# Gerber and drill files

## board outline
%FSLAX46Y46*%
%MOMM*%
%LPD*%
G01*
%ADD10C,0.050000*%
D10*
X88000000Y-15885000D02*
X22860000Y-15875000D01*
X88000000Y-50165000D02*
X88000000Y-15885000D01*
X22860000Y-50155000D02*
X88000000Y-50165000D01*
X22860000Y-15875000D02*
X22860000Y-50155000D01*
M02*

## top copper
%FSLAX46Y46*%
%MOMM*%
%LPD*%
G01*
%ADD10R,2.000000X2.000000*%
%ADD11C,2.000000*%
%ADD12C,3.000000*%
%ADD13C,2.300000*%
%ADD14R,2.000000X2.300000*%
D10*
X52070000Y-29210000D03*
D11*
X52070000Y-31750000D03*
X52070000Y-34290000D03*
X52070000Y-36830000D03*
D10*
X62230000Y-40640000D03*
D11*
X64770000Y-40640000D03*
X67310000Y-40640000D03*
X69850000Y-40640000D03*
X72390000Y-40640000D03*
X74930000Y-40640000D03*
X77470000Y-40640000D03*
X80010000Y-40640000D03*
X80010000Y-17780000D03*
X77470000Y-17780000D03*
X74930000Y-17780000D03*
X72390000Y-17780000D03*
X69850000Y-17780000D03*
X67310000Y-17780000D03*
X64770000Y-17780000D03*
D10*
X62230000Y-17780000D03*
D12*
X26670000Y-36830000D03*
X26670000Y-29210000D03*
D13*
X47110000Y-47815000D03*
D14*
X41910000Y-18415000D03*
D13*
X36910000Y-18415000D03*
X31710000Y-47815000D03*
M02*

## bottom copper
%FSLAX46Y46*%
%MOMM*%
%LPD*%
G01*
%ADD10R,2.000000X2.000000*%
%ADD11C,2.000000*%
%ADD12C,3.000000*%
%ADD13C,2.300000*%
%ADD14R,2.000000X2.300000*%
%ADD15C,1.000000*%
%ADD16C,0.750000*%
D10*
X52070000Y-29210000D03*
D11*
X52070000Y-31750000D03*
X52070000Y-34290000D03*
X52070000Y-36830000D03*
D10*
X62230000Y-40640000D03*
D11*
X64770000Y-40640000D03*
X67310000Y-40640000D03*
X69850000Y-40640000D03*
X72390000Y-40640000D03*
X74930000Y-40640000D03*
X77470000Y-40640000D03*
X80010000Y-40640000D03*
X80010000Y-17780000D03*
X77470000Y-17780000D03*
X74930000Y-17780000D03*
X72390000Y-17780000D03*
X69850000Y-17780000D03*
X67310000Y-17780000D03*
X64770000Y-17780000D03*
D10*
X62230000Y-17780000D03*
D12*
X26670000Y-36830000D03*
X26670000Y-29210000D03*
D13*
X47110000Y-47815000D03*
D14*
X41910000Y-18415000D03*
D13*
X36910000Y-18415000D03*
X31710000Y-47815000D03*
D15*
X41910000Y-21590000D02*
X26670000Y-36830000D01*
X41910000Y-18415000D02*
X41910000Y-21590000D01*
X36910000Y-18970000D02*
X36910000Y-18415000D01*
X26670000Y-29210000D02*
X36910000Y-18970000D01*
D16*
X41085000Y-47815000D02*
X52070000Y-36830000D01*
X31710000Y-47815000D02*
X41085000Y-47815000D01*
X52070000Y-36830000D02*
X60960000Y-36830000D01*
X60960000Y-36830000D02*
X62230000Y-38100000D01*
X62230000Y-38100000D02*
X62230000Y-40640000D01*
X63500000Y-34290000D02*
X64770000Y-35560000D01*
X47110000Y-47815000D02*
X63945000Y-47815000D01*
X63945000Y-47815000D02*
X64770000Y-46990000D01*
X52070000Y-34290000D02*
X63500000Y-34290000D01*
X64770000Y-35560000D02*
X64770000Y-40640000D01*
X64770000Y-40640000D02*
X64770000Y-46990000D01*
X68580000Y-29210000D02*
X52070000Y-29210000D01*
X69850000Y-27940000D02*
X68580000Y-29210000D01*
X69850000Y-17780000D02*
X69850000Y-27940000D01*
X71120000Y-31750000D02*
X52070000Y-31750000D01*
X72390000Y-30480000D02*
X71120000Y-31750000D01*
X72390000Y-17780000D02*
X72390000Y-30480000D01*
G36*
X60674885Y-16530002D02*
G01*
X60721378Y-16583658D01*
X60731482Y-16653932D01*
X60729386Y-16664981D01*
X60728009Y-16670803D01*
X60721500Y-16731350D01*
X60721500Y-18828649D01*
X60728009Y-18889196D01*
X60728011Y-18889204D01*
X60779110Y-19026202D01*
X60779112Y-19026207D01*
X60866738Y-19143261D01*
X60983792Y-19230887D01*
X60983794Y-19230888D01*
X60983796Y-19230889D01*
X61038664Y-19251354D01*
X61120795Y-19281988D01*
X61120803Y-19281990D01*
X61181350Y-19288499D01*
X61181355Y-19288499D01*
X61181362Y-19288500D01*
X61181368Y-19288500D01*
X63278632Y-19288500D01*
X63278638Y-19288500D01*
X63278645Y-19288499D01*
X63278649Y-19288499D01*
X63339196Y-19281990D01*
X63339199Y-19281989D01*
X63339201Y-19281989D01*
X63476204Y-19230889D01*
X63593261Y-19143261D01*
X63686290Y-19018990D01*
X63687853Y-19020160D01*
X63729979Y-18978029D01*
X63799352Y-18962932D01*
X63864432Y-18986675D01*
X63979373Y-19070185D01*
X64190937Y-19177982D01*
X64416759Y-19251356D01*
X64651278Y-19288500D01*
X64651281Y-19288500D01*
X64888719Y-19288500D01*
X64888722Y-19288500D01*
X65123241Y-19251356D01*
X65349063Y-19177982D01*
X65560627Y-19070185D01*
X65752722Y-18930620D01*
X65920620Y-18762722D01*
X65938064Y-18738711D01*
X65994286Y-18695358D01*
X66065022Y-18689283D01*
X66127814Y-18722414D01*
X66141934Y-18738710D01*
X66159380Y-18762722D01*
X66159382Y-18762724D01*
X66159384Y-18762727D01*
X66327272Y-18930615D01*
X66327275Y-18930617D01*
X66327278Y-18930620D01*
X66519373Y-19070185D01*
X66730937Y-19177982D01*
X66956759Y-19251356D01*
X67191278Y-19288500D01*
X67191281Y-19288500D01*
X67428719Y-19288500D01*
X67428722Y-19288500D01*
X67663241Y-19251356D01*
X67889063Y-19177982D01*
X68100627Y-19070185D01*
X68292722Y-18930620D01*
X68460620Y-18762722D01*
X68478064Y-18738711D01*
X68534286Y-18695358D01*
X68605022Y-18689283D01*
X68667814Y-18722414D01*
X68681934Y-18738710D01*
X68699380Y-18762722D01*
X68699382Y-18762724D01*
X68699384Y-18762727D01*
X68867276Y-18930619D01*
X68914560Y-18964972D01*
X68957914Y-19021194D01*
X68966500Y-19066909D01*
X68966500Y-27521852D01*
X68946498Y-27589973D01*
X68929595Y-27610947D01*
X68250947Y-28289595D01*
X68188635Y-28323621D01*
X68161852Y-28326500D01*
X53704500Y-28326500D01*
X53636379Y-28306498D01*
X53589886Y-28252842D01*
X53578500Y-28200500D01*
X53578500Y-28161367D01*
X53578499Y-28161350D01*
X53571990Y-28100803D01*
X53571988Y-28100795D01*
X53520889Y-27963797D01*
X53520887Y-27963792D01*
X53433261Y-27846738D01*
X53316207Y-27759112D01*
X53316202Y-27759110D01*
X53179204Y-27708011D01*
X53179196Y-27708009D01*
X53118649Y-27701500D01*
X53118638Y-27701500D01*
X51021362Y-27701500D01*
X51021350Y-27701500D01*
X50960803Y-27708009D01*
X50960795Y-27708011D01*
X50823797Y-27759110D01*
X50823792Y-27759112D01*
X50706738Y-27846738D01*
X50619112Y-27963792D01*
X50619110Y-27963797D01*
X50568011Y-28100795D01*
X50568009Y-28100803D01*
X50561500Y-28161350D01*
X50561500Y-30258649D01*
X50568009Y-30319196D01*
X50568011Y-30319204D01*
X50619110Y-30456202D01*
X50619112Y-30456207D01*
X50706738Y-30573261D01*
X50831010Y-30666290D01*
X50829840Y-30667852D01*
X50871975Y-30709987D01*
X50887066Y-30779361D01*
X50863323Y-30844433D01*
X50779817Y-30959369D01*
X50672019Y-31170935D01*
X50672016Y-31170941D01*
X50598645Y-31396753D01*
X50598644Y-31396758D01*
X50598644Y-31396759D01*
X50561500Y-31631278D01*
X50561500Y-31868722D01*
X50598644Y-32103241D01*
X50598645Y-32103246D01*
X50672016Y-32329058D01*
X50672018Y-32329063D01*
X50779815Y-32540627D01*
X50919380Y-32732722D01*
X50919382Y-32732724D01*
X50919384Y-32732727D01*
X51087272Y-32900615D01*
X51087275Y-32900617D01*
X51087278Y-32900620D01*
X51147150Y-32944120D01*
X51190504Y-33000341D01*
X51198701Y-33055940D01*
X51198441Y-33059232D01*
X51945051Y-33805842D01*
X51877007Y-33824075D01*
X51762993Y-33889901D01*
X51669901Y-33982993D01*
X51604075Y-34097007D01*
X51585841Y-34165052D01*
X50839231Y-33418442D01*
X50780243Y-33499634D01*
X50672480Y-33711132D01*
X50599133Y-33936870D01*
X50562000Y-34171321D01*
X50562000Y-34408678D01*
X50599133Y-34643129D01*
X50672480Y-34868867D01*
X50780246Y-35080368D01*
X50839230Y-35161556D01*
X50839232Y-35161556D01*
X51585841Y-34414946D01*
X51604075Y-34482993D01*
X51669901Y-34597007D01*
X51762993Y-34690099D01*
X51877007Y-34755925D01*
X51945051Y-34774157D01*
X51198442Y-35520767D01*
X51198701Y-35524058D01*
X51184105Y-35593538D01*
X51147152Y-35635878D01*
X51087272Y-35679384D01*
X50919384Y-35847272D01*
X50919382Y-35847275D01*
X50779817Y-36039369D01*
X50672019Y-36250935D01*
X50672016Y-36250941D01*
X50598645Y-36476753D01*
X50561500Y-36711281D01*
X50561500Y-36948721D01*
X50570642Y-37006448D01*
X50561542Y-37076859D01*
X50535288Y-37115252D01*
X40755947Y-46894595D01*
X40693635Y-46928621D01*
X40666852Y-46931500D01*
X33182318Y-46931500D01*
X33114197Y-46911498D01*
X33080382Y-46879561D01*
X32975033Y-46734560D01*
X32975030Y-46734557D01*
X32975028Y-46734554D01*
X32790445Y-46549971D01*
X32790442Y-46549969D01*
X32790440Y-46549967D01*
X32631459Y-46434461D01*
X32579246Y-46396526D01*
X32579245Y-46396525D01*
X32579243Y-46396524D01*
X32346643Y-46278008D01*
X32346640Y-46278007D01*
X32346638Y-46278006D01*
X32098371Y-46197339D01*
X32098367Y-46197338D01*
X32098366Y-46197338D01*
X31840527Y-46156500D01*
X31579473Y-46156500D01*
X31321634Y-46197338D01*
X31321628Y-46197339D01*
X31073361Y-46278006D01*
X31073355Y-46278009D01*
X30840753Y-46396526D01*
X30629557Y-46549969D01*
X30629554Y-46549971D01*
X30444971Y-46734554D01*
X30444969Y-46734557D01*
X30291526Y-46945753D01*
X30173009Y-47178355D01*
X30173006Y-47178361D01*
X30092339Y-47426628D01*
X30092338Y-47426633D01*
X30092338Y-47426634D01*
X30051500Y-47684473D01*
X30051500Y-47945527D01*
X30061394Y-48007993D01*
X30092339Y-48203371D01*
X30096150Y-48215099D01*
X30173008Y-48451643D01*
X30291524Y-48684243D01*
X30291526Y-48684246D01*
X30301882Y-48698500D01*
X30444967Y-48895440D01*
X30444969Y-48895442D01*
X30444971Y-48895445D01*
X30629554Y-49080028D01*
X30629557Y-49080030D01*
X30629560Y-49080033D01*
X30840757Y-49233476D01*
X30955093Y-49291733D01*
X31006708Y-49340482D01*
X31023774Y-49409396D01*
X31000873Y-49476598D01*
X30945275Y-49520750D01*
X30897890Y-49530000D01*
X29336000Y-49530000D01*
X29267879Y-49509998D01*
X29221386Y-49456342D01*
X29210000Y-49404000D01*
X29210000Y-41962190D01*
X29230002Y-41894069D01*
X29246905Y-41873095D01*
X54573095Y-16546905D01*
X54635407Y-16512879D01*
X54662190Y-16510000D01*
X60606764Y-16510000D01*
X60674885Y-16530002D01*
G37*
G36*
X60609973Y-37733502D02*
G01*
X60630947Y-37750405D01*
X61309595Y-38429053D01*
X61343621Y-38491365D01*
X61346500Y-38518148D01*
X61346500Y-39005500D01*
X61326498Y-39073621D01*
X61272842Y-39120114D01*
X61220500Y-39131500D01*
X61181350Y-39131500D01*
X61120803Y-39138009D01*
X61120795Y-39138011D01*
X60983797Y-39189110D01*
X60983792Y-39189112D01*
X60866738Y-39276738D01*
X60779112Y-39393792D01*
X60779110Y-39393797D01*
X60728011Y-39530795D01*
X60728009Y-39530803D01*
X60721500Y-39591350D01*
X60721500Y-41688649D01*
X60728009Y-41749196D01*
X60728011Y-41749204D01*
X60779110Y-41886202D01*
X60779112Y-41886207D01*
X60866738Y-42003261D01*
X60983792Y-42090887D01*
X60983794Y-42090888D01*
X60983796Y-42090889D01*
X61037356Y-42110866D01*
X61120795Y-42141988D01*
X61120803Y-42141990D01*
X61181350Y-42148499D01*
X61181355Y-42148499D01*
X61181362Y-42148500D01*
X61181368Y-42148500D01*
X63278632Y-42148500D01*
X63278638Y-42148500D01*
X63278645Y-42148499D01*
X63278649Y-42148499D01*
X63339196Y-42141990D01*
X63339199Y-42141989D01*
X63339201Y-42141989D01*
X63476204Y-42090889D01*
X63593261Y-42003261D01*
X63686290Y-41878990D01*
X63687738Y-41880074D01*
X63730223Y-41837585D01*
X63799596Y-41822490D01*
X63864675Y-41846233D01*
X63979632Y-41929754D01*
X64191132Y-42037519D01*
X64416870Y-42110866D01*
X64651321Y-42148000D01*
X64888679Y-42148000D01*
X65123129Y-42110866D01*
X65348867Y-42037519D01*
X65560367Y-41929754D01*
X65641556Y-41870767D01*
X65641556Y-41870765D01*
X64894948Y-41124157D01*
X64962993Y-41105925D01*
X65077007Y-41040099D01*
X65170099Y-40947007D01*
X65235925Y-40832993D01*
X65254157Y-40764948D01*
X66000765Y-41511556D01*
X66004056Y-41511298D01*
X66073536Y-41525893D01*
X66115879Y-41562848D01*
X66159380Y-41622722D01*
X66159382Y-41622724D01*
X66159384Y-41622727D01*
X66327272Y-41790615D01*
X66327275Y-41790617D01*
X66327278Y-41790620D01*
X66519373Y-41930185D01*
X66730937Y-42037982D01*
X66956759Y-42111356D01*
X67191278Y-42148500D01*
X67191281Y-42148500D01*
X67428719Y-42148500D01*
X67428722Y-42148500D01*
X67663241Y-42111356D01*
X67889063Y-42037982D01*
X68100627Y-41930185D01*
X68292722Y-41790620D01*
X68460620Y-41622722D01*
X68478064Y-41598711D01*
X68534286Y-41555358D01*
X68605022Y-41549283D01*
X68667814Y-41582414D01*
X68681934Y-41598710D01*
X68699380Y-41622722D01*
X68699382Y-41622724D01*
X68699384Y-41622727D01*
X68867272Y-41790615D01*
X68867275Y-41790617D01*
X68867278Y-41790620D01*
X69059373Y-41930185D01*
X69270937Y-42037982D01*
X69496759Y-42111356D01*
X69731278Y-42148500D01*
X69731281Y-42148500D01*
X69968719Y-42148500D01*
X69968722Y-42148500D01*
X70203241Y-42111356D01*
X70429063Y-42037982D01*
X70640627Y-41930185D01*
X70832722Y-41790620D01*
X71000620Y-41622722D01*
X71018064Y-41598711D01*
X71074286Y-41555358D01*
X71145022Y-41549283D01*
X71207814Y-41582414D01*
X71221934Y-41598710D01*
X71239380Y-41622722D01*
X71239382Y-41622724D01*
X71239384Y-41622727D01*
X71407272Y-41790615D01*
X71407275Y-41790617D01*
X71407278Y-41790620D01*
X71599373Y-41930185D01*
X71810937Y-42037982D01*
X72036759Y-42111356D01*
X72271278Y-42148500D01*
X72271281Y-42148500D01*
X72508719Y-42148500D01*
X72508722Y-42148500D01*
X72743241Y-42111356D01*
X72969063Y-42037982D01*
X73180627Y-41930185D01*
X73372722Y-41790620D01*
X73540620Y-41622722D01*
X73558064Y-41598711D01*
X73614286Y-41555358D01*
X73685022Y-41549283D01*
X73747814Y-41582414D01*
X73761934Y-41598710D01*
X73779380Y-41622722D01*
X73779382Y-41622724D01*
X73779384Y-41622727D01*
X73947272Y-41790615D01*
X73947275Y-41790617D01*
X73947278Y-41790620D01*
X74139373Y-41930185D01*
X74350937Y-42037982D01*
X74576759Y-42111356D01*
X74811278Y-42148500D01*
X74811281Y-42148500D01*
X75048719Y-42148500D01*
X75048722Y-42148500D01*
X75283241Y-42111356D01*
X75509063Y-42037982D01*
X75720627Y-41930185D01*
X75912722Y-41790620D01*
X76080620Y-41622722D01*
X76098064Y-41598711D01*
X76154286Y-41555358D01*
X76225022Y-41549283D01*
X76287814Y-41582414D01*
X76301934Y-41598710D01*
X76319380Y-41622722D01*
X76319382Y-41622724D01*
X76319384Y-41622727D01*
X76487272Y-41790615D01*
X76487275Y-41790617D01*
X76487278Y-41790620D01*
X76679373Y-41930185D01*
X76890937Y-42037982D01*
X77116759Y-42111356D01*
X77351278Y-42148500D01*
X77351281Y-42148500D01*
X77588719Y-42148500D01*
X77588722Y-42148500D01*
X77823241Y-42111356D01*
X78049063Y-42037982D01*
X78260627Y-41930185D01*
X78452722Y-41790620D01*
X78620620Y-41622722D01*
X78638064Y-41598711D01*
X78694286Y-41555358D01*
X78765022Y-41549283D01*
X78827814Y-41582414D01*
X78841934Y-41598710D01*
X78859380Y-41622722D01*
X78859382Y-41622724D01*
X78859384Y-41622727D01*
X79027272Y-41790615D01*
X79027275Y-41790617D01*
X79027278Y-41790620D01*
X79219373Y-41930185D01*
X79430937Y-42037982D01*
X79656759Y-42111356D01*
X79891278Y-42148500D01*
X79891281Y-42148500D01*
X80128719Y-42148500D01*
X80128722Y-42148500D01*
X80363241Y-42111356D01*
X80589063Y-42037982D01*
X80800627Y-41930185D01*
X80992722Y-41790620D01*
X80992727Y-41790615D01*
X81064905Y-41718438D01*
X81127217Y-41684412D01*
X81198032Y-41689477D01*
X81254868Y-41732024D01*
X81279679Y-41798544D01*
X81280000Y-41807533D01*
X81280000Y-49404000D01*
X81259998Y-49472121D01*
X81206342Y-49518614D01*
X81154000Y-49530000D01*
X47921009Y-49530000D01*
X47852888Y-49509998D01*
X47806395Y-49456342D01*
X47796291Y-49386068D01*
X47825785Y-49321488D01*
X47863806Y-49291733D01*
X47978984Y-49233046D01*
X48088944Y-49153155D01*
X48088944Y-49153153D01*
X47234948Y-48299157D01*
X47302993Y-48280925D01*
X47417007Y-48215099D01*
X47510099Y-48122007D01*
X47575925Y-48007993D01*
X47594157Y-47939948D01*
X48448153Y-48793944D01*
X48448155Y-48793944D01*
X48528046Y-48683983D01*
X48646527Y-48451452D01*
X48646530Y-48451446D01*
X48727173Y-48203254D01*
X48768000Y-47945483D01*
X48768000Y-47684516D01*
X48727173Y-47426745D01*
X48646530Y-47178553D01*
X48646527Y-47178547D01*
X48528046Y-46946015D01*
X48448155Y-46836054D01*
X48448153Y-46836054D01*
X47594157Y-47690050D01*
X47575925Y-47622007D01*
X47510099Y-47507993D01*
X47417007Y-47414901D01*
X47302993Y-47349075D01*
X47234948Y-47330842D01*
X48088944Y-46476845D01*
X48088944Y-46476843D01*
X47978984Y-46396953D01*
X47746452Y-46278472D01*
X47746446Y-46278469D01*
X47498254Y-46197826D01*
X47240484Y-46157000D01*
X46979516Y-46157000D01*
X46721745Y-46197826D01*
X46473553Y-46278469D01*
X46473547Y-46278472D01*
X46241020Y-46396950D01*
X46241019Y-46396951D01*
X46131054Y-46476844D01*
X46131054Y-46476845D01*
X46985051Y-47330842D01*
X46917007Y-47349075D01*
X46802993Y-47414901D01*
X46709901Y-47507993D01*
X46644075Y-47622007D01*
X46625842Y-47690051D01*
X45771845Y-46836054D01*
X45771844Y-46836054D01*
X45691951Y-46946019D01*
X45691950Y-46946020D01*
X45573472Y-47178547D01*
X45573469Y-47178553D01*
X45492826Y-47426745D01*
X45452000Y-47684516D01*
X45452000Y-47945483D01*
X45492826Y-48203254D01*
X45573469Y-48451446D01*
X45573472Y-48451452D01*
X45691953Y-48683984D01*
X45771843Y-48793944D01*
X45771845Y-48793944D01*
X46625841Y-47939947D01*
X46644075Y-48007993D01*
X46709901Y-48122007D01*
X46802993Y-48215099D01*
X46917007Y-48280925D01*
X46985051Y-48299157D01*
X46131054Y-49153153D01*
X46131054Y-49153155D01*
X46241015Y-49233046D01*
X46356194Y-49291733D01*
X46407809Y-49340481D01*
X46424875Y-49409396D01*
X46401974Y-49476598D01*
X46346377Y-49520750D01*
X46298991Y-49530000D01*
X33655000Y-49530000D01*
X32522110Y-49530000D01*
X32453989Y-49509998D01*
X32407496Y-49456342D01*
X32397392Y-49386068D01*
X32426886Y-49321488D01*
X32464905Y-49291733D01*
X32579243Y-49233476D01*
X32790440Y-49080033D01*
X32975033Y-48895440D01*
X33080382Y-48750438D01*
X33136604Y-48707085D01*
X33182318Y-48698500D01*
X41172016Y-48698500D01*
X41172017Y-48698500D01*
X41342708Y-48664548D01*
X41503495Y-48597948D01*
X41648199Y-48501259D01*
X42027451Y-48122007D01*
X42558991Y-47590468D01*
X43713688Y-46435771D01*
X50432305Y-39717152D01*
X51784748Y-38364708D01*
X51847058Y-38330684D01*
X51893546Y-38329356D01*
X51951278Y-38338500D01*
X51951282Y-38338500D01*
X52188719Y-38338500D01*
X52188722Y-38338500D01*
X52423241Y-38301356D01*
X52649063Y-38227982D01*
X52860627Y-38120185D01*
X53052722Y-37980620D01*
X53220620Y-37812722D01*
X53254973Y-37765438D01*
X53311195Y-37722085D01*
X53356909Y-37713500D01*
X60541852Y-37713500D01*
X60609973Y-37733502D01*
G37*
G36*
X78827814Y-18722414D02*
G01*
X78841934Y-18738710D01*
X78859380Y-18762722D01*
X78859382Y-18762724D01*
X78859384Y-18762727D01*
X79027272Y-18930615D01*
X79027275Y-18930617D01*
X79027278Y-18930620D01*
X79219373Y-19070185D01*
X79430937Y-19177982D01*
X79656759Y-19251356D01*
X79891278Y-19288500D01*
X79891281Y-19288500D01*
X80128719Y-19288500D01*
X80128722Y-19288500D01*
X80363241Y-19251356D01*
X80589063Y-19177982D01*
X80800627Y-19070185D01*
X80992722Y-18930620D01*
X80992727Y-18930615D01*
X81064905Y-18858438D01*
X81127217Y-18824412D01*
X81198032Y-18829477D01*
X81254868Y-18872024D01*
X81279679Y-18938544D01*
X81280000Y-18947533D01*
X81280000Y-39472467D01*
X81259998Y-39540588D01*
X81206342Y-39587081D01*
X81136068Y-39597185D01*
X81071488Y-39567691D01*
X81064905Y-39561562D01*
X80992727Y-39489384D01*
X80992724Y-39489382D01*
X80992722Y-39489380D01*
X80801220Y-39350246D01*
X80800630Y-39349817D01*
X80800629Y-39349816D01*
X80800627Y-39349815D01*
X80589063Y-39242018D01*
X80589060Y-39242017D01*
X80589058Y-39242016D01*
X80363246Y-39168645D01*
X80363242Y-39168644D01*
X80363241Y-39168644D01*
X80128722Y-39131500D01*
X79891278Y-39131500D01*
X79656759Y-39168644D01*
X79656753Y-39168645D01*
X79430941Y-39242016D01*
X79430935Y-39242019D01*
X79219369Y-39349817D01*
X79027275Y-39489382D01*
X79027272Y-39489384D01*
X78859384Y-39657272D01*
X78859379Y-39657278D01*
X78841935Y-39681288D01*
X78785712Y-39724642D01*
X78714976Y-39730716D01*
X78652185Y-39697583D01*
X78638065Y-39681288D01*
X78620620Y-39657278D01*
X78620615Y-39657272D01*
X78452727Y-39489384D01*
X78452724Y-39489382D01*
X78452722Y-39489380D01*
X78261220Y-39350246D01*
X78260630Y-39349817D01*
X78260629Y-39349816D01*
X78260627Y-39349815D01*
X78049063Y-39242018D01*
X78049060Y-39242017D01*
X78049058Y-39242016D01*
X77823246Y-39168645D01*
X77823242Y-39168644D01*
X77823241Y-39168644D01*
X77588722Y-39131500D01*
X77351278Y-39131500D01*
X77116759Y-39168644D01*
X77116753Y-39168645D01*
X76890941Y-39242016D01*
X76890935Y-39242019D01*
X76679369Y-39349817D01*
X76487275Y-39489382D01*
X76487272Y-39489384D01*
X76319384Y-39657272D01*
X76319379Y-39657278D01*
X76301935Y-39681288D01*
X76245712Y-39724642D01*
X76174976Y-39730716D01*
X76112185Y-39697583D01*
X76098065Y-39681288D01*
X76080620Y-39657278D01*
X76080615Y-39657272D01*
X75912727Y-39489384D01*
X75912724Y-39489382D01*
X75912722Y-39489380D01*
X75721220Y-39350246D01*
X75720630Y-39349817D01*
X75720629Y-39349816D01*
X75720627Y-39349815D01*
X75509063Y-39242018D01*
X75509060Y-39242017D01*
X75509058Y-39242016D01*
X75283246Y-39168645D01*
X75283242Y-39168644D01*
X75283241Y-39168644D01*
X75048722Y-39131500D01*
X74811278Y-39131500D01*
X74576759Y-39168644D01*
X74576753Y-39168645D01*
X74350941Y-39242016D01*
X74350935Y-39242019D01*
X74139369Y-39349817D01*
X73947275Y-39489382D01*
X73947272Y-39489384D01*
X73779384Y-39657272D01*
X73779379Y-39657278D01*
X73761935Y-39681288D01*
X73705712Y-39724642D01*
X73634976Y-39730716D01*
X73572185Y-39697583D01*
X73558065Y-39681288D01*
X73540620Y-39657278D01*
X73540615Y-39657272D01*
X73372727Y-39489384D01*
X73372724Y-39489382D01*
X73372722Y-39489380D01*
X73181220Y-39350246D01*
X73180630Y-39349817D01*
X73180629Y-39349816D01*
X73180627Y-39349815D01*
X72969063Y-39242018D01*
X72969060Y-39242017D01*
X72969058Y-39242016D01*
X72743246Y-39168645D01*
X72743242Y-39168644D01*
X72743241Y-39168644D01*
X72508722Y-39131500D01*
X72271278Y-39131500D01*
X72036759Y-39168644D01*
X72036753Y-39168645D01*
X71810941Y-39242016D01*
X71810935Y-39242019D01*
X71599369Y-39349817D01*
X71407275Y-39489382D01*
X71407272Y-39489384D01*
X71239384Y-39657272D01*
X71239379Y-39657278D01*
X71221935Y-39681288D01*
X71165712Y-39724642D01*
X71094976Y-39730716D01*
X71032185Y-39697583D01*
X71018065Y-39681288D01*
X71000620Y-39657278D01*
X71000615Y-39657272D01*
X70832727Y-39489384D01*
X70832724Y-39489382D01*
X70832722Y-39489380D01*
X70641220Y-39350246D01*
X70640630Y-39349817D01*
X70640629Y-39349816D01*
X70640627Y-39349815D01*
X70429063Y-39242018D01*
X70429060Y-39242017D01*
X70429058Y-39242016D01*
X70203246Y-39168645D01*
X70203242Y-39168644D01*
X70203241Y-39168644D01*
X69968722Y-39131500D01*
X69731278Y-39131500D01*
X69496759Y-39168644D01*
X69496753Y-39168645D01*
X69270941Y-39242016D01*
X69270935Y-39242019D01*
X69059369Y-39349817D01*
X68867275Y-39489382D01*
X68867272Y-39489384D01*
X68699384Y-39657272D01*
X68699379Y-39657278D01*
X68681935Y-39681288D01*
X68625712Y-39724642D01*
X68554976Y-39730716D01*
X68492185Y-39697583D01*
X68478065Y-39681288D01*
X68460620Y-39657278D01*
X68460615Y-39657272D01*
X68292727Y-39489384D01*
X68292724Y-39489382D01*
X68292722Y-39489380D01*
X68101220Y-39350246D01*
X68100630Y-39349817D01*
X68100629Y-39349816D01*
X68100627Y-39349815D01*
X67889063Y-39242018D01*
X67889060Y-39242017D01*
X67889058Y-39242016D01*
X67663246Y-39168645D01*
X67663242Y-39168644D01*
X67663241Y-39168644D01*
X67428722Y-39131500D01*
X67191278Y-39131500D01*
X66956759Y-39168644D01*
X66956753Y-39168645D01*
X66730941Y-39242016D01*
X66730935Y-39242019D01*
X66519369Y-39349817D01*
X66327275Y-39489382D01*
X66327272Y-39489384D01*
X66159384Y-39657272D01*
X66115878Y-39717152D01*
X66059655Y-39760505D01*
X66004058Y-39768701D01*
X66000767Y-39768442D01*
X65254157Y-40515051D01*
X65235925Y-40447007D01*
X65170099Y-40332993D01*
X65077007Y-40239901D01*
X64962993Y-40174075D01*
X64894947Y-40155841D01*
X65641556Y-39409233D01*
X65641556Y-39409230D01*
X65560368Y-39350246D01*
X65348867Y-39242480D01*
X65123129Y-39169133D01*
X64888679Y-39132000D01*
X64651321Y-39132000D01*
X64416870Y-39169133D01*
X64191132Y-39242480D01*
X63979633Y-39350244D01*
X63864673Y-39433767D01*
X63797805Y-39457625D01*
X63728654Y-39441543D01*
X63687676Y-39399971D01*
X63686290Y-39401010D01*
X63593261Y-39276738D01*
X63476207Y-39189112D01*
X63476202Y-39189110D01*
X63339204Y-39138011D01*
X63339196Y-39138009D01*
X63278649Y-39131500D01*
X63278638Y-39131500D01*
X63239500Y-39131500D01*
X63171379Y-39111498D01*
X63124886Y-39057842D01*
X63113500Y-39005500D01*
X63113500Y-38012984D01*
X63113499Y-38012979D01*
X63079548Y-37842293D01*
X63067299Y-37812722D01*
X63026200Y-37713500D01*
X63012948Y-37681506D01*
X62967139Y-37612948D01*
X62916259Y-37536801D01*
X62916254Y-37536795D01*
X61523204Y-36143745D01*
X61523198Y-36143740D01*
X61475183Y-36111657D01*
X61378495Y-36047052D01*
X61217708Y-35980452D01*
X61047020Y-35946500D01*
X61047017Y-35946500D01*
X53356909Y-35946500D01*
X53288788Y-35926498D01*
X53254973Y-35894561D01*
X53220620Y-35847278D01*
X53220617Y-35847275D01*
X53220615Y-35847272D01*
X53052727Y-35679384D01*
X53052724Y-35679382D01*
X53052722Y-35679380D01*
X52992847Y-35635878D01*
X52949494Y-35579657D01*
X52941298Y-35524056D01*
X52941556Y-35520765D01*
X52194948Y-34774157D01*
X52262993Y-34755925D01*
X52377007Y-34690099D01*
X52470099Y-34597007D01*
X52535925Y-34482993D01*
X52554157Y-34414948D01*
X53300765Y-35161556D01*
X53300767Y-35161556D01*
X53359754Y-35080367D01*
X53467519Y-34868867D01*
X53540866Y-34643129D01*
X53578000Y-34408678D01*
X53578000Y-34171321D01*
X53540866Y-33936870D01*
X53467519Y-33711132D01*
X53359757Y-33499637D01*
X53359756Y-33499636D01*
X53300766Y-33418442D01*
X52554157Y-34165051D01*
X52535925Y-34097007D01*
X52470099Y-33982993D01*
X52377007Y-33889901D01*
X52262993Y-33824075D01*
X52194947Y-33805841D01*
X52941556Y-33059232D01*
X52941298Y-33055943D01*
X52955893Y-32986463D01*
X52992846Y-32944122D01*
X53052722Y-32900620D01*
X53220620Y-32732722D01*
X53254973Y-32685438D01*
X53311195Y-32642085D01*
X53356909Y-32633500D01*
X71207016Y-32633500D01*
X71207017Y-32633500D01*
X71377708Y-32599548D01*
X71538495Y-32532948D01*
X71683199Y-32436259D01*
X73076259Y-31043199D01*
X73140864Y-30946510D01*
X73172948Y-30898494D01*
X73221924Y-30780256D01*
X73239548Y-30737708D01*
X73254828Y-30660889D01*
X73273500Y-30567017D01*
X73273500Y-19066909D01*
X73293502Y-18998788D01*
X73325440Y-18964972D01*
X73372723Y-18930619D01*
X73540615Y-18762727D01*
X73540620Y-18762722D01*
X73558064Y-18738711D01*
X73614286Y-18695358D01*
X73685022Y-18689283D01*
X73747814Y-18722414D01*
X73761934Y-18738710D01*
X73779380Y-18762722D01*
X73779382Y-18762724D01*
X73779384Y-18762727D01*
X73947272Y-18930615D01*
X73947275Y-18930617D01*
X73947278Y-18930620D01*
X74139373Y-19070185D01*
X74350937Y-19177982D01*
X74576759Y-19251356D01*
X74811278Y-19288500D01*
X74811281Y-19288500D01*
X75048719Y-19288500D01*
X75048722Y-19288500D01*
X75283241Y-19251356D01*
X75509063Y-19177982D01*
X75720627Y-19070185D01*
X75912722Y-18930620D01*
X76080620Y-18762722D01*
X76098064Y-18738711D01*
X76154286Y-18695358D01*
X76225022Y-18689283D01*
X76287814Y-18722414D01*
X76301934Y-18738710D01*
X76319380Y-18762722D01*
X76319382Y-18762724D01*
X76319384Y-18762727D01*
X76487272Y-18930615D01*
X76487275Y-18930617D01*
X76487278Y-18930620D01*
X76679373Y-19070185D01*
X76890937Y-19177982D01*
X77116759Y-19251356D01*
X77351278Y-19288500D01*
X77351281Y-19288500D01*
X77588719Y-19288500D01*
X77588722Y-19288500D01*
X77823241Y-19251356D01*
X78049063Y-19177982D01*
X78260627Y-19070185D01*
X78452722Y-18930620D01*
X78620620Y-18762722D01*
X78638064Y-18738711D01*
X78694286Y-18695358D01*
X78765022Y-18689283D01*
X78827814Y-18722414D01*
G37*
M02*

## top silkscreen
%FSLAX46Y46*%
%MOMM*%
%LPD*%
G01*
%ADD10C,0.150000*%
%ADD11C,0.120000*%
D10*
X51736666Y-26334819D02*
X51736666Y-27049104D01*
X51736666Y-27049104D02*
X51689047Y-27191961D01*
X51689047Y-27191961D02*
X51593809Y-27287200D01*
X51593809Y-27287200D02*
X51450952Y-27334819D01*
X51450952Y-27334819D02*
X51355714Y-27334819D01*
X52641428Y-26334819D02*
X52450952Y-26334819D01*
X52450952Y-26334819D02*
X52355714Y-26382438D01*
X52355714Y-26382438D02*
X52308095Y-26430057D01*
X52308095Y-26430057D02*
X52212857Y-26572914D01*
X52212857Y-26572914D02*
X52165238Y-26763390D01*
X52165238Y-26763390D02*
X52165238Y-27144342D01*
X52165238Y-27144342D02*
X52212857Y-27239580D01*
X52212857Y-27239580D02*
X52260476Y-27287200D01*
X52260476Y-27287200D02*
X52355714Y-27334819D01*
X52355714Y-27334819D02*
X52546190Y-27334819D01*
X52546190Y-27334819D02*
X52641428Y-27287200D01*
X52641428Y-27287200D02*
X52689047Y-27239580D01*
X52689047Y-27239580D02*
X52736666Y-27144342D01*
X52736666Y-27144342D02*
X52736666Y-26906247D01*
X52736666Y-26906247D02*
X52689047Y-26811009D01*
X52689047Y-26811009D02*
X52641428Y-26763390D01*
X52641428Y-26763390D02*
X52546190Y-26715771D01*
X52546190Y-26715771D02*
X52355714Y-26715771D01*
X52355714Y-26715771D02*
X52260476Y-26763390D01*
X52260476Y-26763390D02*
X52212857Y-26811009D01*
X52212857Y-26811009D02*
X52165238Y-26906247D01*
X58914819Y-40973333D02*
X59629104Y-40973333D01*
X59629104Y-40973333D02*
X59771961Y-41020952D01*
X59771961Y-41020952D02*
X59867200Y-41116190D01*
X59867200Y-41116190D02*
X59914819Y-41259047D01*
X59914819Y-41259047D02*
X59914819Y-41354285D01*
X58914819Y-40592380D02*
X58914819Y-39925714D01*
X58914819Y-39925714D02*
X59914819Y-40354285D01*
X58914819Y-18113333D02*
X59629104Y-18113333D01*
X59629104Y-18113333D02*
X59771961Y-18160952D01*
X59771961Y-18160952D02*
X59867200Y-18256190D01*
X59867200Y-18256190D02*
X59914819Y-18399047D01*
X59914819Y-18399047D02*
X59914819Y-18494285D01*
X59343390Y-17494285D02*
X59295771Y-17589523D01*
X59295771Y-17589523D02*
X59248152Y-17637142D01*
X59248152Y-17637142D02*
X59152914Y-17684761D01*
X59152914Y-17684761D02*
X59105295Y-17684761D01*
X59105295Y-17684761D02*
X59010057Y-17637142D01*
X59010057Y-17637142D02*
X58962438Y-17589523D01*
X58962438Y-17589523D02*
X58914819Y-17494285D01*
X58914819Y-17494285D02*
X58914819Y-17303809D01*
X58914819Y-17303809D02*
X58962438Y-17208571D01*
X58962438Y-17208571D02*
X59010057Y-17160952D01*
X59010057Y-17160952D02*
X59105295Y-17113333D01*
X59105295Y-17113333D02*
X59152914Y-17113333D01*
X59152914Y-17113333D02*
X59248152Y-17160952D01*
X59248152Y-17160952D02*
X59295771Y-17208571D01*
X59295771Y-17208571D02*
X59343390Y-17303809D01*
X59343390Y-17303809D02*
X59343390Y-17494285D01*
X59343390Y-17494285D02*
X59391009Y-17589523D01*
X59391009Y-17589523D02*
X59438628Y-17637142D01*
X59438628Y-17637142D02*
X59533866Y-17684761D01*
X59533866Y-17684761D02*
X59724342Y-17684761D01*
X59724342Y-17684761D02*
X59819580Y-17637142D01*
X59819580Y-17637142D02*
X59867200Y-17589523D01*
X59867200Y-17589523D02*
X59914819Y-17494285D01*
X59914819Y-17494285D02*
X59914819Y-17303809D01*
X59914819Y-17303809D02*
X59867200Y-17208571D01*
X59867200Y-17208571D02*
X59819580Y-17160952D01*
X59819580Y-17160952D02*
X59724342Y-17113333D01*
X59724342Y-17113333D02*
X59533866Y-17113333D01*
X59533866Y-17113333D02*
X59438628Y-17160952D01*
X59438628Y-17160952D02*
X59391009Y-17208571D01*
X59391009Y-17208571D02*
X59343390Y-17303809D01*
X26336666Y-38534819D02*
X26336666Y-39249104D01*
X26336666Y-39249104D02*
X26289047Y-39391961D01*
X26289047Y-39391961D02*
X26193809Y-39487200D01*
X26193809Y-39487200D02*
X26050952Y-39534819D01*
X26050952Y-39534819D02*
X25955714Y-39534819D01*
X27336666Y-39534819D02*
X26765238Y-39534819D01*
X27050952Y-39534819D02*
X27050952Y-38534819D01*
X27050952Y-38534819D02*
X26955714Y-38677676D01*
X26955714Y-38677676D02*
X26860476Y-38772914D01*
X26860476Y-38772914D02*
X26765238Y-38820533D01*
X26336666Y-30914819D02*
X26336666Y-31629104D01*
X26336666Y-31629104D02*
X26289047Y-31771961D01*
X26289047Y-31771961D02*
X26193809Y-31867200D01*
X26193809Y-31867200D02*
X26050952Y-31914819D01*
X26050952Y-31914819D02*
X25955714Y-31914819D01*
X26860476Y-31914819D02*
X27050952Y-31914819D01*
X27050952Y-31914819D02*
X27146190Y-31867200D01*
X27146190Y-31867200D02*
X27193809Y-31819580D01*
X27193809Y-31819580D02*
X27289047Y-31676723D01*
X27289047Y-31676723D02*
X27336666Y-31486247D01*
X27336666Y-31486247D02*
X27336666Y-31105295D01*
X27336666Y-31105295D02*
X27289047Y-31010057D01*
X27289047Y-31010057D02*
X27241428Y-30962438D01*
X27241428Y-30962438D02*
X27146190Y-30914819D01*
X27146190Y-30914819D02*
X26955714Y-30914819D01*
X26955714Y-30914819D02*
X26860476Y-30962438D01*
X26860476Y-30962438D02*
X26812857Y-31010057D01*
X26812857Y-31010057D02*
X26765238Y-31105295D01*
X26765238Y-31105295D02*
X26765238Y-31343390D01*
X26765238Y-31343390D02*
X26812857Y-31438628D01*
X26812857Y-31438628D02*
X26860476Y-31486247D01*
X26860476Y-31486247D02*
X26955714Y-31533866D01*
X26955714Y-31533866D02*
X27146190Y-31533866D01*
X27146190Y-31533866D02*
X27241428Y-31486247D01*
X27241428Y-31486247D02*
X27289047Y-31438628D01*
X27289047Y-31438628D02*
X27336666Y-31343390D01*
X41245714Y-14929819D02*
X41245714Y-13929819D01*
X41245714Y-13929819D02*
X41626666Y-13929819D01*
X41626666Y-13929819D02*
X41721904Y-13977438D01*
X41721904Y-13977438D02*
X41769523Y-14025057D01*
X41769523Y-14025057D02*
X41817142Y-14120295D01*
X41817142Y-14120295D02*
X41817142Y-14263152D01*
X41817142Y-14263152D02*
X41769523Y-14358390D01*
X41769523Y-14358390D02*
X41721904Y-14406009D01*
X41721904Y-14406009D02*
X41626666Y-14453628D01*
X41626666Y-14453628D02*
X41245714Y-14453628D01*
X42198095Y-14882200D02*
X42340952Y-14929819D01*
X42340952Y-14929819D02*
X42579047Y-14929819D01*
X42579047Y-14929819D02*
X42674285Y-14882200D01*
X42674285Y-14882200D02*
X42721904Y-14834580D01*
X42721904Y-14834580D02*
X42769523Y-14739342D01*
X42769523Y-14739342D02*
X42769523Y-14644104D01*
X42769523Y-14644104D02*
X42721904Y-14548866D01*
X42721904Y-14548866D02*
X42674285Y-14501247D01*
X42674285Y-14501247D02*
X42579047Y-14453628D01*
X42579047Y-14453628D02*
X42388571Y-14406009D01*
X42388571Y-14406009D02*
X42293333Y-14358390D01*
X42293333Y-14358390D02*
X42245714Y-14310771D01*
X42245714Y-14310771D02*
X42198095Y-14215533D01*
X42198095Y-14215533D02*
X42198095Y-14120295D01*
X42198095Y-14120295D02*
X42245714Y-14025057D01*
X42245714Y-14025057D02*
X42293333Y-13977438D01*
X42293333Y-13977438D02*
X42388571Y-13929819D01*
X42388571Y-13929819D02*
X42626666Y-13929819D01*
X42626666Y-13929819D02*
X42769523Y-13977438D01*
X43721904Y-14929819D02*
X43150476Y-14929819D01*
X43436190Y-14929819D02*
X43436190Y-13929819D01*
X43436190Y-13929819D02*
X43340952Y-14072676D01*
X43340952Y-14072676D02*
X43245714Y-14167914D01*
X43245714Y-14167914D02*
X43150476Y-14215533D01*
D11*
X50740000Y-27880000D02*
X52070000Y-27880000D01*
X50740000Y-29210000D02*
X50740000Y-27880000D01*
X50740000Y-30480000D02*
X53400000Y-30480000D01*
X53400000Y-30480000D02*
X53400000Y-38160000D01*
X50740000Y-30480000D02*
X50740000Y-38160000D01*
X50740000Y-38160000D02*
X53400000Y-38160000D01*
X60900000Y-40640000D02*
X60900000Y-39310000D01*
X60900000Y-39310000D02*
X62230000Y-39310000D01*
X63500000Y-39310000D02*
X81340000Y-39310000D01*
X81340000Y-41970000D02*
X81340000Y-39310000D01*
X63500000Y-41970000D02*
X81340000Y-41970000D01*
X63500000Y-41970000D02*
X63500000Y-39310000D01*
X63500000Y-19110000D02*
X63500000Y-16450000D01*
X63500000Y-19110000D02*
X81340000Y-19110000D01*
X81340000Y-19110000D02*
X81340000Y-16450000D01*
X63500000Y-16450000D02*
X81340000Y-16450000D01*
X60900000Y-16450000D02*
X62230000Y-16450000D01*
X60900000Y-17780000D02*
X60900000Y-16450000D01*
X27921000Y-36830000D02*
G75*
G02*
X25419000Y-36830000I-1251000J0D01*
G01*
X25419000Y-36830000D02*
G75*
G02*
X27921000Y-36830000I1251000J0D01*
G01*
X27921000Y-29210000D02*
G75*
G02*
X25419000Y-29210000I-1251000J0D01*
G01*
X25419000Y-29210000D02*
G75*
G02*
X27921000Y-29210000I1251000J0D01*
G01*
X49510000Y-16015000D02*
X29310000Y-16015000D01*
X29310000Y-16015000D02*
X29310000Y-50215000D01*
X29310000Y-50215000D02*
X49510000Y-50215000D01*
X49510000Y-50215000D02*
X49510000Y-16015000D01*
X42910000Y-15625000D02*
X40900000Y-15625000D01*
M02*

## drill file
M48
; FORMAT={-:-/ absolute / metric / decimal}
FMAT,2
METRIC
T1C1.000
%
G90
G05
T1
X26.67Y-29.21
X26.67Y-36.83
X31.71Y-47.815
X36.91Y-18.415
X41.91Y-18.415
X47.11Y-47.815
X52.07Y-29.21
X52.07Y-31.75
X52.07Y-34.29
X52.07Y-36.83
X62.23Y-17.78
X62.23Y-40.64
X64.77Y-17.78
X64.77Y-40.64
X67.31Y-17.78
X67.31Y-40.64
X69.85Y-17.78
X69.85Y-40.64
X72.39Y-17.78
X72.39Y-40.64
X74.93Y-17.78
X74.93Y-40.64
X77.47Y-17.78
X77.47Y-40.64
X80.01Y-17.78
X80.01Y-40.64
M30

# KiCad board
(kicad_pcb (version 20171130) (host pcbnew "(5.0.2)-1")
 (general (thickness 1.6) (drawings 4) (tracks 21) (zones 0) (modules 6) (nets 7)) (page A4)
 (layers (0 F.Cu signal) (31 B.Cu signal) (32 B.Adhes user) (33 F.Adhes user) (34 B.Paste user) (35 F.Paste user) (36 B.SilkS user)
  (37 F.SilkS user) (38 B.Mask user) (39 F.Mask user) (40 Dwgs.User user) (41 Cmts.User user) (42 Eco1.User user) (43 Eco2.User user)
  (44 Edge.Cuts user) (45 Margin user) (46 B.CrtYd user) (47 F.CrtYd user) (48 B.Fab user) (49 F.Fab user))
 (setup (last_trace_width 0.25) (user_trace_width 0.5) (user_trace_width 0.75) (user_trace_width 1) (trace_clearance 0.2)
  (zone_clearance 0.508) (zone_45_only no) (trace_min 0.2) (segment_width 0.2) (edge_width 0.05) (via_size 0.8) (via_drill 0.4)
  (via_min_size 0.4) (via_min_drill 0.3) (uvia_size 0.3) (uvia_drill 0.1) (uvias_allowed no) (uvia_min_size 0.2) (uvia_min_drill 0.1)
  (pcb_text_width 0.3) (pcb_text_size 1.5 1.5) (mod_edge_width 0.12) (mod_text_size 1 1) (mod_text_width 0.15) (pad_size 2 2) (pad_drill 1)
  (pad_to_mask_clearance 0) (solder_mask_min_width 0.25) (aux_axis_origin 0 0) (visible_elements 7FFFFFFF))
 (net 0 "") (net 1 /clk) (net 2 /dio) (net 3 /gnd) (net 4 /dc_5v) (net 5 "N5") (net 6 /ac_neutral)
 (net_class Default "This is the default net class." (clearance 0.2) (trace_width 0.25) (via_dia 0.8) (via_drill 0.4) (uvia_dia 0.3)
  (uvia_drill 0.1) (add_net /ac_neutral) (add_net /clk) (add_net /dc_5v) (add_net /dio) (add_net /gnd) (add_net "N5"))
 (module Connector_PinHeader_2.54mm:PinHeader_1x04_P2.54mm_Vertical (layer F.Cu) (at 52.07 29.21)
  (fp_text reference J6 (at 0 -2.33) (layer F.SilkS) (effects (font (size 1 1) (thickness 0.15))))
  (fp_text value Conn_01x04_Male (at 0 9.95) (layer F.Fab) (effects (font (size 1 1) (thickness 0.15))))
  (fp_line (start -1.33 -1.33) (end 0 -1.33) (layer F.SilkS) (width 0.12))
  (fp_line (start -1.33 0) (end -1.33 -1.33) (layer F.SilkS) (width 0.12))
  (fp_line (start -1.33 1.27) (end 1.33 1.27) (layer F.SilkS) (width 0.12))
  (fp_line (start 1.33 1.27) (end 1.33 8.95) (layer F.SilkS) (width 0.12))
  (fp_line (start -1.33 1.27) (end -1.33 8.95) (layer F.SilkS) (width 0.12))
  (fp_line (start -1.33 8.95) (end 1.33 8.95) (layer F.SilkS) (width 0.12))
  (pad 1 thru_hole rect (at 0 0) (size 2 2) (drill 1) (layers *.Cu *.Mask) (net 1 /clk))
  (pad 2 thru_hole circle (at 0 2.54) (size 2 2) (drill 1) (layers *.Cu *.Mask) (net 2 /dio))
  (pad 3 thru_hole circle (at 0 5.08) (size 2 2) (drill 1) (layers *.Cu *.Mask) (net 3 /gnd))
  (pad 4 thru_hole circle (at 0 7.62) (size 2 2) (drill 1) (layers *.Cu *.Mask) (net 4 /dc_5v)))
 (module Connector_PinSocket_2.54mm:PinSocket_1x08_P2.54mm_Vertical (layer F.Cu) (at 62.23 40.64 90)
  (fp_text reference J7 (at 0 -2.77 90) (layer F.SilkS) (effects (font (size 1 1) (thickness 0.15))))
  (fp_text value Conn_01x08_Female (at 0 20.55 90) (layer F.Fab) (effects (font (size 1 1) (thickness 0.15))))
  (fp_line (start 0 -1.33) (end 1.33 -1.33) (layer F.SilkS) (width 0.12))
  (fp_line (start 1.33 -1.33) (end 1.33 0) (layer F.SilkS) (width 0.12))
  (fp_line (start 1.33 1.27) (end 1.33 19.11) (layer F.SilkS) (width 0.12))
  (fp_line (start -1.33 19.11) (end 1.33 19.11) (layer F.SilkS) (width 0.12))
  (fp_line (start -1.33 1.27) (end -1.33 19.11) (layer F.SilkS) (width 0.12))
  (fp_line (start -1.33 1.27) (end 1.33 1.27) (layer F.SilkS) (width 0.12))
  (pad 1 thru_hole rect (at 0 0 90) (size 2 2) (drill 1) (layers *.Cu *.Mask) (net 4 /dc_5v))
  (pad 2 thru_hole circle (at 0 2.54 90) (size 2 2) (drill 1) (layers *.Cu *.Mask) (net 3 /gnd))
  (pad 3 thru_hole circle (at 0 5.08 90) (size 2 2) (drill 1) (layers *.Cu *.Mask))
  (pad 4 thru_hole circle (at 0 7.62 90) (size 2 2) (drill 1) (layers *.Cu *.Mask))
  (pad 5 thru_hole circle (at 0 10.16 90) (size 2 2) (drill 1) (layers *.Cu *.Mask))
  (pad 6 thru_hole circle (at 0 12.7 90) (size 2 2) (drill 1) (layers *.Cu *.Mask))
  (pad 7 thru_hole circle (at 0 15.24 90) (size 2 2) (drill 1) (layers *.Cu *.Mask))
  (pad 8 thru_hole circle (at 0 17.78 90) (size 2 2) (drill 1) (layers *.Cu *.Mask)))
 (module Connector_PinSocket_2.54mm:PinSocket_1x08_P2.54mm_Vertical (layer F.Cu) (at 62.23 17.78 90)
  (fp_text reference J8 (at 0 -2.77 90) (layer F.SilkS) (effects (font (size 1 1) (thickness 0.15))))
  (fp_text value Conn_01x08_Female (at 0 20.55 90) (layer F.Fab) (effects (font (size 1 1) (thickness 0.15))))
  (fp_line (start -1.33 1.27) (end 1.33 1.27) (layer F.SilkS) (width 0.12))
  (fp_line (start -1.33 1.27) (end -1.33 19.11) (layer F.SilkS) (width 0.12))
  (fp_line (start -1.33 19.11) (end 1.33 19.11) (layer F.SilkS) (width 0.12))
  (fp_line (start 1.33 1.27) (end 1.33 19.11) (layer F.SilkS) (width 0.12))
  (fp_line (start 1.33 -1.33) (end 1.33 0) (layer F.SilkS) (width 0.12))
  (fp_line (start 0 -1.33) (end 1.33 -1.33) (layer F.SilkS) (width 0.12))
  (pad 8 thru_hole circle (at 0 17.78 90) (size 2 2) (drill 1) (layers *.Cu *.Mask))
  (pad 7 thru_hole circle (at 0 15.24 90) (size 2 2) (drill 1) (layers *.Cu *.Mask))
  (pad 6 thru_hole circle (at 0 12.7 90) (size 2 2) (drill 1) (layers *.Cu *.Mask))
  (pad 5 thru_hole circle (at 0 10.16 90) (size 2 2) (drill 1) (layers *.Cu *.Mask) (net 2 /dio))
  (pad 4 thru_hole circle (at 0 7.62 90) (size 2 2) (drill 1) (layers *.Cu *.Mask) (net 1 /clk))
  (pad 3 thru_hole circle (at 0 5.08 90) (size 2 2) (drill 1) (layers *.Cu *.Mask))
  (pad 2 thru_hole circle (at 0 2.54 90) (size 2 2) (drill 1) (layers *.Cu *.Mask))
  (pad 1 thru_hole rect (at 0 0 90) (size 2 2) (drill 1) (layers *.Cu *.Mask)))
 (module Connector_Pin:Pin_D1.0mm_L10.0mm (layer F.Cu) (at 26.67 36.83)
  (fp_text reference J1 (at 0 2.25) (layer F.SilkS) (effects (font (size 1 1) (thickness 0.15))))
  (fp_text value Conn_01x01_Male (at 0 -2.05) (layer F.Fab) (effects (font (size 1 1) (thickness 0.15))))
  (fp_circle (center 0 0) (end 1.25 0.05) (layer F.SilkS) (width 0.12))
  (pad 1 thru_hole circle (at 0 0) (size 3 3) (drill 1) (layers *.Cu *.Mask) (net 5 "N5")))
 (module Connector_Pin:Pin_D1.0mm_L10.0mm (layer F.Cu) (at 26.67 29.21)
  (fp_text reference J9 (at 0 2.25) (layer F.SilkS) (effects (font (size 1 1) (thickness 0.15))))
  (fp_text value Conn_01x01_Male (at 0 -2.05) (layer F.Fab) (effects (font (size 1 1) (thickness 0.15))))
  (fp_circle (center 0 0) (end 1.25 0.05) (layer F.SilkS) (width 0.12))
  (pad 1 thru_hole circle (at 0 0) (size 3 3) (drill 1) (layers *.Cu *.Mask) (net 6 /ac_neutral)))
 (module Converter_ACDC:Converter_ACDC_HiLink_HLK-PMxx (layer F.Cu) (at 41.91 18.415 270)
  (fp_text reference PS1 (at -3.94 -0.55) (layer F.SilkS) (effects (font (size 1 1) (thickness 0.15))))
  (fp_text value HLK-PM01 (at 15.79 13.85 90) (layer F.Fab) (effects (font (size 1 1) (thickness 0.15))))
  (fp_line (start -2.4 -7.6) (end -2.4 12.6) (layer F.SilkS) (width 0.12))
  (fp_line (start -2.4 12.6) (end 31.8 12.6) (layer F.SilkS) (width 0.12))
  (fp_line (start 31.8 12.6) (end 31.8 -7.6) (layer F.SilkS) (width 0.12))
  (fp_line (start 31.8 -7.6) (end -2.4 -7.6) (layer F.SilkS) (width 0.12))
  (fp_line (start -2.79 -1) (end -2.79 1.01) (layer F.SilkS) (width 0.12))
  (pad 3 thru_hole circle (at 29.4 -5.2 270) (size 2.3 2.3) (drill 1) (layers *.Cu *.Mask) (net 3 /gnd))
  (pad 1 thru_hole rect (at 0 0 270) (size 2.3 2) (drill 1) (layers *.Cu *.Mask) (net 5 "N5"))
  (pad 2 thru_hole circle (at 0 5 270) (size 2.3 2.3) (drill 1) (layers *.Cu *.Mask) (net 6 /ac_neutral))
  (pad 4 thru_hole circle (at 29.4 10.2 270) (size 2.3 2.3) (drill 1) (layers *.Cu *.Mask) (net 4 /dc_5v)))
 (gr_line (start 88 15.885) (end 22.86 15.875) (layer Edge.Cuts) (width 0.05))
 (gr_line (start 88 50.165) (end 88 15.885) (layer Edge.Cuts) (width 0.05))
 (gr_line (start 22.86 50.155) (end 88 50.165) (layer Edge.Cuts) (width 0.05))
 (gr_line (start 22.86 15.875) (end 22.86 50.155) (layer Edge.Cuts) (width 0.05))
 (segment (start 41.91 21.59) (end 26.67 36.83) (width 1) (layer B.Cu) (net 5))
 (segment (start 41.91 18.415) (end 41.91 21.59) (width 1) (layer B.Cu) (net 5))
 (segment (start 36.91 18.97) (end 36.91 18.415) (width 1) (layer B.Cu) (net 6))
 (segment (start 26.67 29.21) (end 36.91 18.97) (width 1) (layer B.Cu) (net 6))
 (segment (start 41.085 47.815) (end 52.07 36.83) (width 0.75) (layer B.Cu) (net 4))
 (segment (start 31.71 47.815) (end 41.085 47.815) (width 0.75) (layer B.Cu) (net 4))
 (segment (start 52.07 36.83) (end 60.96 36.83) (width 0.75) (layer B.Cu) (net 4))
 (segment (start 60.96 36.83) (end 62.23 38.1) (width 0.75) (layer B.Cu) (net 4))
 (segment (start 62.23 38.1) (end 62.23 40.64) (width 0.75) (layer B.Cu) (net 4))
 (segment (start 63.5 34.29) (end 64.77 35.56) (width 0.75) (layer B.Cu) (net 3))
 (segment (start 47.11 47.815) (end 63.945 47.815) (width 0.75) (layer B.Cu) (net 3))
 (segment (start 63.945 47.815) (end 64.77 46.99) (width 0.75) (layer B.Cu) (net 3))
 (segment (start 52.07 34.29) (end 63.5 34.29) (width 0.75) (layer B.Cu) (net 3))
 (segment (start 64.77 35.56) (end 64.77 40.64) (width 0.75) (layer B.Cu) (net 3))
 (segment (start 64.77 40.64) (end 64.77 46.99) (width 0.75) (layer B.Cu) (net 3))
 (segment (start 68.58 29.21) (end 52.07 29.21) (width 0.75) (layer B.Cu) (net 1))
 (segment (start 69.85 27.94) (end 68.58 29.21) (width 0.75) (layer B.Cu) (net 1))
 (segment (start 69.85 17.78) (end 69.85 27.94) (width 0.75) (layer B.Cu) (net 1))
 (segment (start 71.12 31.75) (end 52.07 31.75) (width 0.75) (layer B.Cu) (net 2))
 (segment (start 72.39 30.48) (end 71.12 31.75) (width 0.75) (layer B.Cu) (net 2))
 (segment (start 72.39 17.78) (end 72.39 30.48) (width 0.75) (layer B.Cu) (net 2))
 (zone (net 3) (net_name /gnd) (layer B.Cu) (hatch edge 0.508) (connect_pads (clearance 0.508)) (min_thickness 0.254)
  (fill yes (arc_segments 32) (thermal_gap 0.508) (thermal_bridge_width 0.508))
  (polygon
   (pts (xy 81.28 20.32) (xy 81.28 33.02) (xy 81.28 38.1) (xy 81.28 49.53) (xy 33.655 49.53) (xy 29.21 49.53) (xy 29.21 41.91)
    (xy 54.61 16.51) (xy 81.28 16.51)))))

